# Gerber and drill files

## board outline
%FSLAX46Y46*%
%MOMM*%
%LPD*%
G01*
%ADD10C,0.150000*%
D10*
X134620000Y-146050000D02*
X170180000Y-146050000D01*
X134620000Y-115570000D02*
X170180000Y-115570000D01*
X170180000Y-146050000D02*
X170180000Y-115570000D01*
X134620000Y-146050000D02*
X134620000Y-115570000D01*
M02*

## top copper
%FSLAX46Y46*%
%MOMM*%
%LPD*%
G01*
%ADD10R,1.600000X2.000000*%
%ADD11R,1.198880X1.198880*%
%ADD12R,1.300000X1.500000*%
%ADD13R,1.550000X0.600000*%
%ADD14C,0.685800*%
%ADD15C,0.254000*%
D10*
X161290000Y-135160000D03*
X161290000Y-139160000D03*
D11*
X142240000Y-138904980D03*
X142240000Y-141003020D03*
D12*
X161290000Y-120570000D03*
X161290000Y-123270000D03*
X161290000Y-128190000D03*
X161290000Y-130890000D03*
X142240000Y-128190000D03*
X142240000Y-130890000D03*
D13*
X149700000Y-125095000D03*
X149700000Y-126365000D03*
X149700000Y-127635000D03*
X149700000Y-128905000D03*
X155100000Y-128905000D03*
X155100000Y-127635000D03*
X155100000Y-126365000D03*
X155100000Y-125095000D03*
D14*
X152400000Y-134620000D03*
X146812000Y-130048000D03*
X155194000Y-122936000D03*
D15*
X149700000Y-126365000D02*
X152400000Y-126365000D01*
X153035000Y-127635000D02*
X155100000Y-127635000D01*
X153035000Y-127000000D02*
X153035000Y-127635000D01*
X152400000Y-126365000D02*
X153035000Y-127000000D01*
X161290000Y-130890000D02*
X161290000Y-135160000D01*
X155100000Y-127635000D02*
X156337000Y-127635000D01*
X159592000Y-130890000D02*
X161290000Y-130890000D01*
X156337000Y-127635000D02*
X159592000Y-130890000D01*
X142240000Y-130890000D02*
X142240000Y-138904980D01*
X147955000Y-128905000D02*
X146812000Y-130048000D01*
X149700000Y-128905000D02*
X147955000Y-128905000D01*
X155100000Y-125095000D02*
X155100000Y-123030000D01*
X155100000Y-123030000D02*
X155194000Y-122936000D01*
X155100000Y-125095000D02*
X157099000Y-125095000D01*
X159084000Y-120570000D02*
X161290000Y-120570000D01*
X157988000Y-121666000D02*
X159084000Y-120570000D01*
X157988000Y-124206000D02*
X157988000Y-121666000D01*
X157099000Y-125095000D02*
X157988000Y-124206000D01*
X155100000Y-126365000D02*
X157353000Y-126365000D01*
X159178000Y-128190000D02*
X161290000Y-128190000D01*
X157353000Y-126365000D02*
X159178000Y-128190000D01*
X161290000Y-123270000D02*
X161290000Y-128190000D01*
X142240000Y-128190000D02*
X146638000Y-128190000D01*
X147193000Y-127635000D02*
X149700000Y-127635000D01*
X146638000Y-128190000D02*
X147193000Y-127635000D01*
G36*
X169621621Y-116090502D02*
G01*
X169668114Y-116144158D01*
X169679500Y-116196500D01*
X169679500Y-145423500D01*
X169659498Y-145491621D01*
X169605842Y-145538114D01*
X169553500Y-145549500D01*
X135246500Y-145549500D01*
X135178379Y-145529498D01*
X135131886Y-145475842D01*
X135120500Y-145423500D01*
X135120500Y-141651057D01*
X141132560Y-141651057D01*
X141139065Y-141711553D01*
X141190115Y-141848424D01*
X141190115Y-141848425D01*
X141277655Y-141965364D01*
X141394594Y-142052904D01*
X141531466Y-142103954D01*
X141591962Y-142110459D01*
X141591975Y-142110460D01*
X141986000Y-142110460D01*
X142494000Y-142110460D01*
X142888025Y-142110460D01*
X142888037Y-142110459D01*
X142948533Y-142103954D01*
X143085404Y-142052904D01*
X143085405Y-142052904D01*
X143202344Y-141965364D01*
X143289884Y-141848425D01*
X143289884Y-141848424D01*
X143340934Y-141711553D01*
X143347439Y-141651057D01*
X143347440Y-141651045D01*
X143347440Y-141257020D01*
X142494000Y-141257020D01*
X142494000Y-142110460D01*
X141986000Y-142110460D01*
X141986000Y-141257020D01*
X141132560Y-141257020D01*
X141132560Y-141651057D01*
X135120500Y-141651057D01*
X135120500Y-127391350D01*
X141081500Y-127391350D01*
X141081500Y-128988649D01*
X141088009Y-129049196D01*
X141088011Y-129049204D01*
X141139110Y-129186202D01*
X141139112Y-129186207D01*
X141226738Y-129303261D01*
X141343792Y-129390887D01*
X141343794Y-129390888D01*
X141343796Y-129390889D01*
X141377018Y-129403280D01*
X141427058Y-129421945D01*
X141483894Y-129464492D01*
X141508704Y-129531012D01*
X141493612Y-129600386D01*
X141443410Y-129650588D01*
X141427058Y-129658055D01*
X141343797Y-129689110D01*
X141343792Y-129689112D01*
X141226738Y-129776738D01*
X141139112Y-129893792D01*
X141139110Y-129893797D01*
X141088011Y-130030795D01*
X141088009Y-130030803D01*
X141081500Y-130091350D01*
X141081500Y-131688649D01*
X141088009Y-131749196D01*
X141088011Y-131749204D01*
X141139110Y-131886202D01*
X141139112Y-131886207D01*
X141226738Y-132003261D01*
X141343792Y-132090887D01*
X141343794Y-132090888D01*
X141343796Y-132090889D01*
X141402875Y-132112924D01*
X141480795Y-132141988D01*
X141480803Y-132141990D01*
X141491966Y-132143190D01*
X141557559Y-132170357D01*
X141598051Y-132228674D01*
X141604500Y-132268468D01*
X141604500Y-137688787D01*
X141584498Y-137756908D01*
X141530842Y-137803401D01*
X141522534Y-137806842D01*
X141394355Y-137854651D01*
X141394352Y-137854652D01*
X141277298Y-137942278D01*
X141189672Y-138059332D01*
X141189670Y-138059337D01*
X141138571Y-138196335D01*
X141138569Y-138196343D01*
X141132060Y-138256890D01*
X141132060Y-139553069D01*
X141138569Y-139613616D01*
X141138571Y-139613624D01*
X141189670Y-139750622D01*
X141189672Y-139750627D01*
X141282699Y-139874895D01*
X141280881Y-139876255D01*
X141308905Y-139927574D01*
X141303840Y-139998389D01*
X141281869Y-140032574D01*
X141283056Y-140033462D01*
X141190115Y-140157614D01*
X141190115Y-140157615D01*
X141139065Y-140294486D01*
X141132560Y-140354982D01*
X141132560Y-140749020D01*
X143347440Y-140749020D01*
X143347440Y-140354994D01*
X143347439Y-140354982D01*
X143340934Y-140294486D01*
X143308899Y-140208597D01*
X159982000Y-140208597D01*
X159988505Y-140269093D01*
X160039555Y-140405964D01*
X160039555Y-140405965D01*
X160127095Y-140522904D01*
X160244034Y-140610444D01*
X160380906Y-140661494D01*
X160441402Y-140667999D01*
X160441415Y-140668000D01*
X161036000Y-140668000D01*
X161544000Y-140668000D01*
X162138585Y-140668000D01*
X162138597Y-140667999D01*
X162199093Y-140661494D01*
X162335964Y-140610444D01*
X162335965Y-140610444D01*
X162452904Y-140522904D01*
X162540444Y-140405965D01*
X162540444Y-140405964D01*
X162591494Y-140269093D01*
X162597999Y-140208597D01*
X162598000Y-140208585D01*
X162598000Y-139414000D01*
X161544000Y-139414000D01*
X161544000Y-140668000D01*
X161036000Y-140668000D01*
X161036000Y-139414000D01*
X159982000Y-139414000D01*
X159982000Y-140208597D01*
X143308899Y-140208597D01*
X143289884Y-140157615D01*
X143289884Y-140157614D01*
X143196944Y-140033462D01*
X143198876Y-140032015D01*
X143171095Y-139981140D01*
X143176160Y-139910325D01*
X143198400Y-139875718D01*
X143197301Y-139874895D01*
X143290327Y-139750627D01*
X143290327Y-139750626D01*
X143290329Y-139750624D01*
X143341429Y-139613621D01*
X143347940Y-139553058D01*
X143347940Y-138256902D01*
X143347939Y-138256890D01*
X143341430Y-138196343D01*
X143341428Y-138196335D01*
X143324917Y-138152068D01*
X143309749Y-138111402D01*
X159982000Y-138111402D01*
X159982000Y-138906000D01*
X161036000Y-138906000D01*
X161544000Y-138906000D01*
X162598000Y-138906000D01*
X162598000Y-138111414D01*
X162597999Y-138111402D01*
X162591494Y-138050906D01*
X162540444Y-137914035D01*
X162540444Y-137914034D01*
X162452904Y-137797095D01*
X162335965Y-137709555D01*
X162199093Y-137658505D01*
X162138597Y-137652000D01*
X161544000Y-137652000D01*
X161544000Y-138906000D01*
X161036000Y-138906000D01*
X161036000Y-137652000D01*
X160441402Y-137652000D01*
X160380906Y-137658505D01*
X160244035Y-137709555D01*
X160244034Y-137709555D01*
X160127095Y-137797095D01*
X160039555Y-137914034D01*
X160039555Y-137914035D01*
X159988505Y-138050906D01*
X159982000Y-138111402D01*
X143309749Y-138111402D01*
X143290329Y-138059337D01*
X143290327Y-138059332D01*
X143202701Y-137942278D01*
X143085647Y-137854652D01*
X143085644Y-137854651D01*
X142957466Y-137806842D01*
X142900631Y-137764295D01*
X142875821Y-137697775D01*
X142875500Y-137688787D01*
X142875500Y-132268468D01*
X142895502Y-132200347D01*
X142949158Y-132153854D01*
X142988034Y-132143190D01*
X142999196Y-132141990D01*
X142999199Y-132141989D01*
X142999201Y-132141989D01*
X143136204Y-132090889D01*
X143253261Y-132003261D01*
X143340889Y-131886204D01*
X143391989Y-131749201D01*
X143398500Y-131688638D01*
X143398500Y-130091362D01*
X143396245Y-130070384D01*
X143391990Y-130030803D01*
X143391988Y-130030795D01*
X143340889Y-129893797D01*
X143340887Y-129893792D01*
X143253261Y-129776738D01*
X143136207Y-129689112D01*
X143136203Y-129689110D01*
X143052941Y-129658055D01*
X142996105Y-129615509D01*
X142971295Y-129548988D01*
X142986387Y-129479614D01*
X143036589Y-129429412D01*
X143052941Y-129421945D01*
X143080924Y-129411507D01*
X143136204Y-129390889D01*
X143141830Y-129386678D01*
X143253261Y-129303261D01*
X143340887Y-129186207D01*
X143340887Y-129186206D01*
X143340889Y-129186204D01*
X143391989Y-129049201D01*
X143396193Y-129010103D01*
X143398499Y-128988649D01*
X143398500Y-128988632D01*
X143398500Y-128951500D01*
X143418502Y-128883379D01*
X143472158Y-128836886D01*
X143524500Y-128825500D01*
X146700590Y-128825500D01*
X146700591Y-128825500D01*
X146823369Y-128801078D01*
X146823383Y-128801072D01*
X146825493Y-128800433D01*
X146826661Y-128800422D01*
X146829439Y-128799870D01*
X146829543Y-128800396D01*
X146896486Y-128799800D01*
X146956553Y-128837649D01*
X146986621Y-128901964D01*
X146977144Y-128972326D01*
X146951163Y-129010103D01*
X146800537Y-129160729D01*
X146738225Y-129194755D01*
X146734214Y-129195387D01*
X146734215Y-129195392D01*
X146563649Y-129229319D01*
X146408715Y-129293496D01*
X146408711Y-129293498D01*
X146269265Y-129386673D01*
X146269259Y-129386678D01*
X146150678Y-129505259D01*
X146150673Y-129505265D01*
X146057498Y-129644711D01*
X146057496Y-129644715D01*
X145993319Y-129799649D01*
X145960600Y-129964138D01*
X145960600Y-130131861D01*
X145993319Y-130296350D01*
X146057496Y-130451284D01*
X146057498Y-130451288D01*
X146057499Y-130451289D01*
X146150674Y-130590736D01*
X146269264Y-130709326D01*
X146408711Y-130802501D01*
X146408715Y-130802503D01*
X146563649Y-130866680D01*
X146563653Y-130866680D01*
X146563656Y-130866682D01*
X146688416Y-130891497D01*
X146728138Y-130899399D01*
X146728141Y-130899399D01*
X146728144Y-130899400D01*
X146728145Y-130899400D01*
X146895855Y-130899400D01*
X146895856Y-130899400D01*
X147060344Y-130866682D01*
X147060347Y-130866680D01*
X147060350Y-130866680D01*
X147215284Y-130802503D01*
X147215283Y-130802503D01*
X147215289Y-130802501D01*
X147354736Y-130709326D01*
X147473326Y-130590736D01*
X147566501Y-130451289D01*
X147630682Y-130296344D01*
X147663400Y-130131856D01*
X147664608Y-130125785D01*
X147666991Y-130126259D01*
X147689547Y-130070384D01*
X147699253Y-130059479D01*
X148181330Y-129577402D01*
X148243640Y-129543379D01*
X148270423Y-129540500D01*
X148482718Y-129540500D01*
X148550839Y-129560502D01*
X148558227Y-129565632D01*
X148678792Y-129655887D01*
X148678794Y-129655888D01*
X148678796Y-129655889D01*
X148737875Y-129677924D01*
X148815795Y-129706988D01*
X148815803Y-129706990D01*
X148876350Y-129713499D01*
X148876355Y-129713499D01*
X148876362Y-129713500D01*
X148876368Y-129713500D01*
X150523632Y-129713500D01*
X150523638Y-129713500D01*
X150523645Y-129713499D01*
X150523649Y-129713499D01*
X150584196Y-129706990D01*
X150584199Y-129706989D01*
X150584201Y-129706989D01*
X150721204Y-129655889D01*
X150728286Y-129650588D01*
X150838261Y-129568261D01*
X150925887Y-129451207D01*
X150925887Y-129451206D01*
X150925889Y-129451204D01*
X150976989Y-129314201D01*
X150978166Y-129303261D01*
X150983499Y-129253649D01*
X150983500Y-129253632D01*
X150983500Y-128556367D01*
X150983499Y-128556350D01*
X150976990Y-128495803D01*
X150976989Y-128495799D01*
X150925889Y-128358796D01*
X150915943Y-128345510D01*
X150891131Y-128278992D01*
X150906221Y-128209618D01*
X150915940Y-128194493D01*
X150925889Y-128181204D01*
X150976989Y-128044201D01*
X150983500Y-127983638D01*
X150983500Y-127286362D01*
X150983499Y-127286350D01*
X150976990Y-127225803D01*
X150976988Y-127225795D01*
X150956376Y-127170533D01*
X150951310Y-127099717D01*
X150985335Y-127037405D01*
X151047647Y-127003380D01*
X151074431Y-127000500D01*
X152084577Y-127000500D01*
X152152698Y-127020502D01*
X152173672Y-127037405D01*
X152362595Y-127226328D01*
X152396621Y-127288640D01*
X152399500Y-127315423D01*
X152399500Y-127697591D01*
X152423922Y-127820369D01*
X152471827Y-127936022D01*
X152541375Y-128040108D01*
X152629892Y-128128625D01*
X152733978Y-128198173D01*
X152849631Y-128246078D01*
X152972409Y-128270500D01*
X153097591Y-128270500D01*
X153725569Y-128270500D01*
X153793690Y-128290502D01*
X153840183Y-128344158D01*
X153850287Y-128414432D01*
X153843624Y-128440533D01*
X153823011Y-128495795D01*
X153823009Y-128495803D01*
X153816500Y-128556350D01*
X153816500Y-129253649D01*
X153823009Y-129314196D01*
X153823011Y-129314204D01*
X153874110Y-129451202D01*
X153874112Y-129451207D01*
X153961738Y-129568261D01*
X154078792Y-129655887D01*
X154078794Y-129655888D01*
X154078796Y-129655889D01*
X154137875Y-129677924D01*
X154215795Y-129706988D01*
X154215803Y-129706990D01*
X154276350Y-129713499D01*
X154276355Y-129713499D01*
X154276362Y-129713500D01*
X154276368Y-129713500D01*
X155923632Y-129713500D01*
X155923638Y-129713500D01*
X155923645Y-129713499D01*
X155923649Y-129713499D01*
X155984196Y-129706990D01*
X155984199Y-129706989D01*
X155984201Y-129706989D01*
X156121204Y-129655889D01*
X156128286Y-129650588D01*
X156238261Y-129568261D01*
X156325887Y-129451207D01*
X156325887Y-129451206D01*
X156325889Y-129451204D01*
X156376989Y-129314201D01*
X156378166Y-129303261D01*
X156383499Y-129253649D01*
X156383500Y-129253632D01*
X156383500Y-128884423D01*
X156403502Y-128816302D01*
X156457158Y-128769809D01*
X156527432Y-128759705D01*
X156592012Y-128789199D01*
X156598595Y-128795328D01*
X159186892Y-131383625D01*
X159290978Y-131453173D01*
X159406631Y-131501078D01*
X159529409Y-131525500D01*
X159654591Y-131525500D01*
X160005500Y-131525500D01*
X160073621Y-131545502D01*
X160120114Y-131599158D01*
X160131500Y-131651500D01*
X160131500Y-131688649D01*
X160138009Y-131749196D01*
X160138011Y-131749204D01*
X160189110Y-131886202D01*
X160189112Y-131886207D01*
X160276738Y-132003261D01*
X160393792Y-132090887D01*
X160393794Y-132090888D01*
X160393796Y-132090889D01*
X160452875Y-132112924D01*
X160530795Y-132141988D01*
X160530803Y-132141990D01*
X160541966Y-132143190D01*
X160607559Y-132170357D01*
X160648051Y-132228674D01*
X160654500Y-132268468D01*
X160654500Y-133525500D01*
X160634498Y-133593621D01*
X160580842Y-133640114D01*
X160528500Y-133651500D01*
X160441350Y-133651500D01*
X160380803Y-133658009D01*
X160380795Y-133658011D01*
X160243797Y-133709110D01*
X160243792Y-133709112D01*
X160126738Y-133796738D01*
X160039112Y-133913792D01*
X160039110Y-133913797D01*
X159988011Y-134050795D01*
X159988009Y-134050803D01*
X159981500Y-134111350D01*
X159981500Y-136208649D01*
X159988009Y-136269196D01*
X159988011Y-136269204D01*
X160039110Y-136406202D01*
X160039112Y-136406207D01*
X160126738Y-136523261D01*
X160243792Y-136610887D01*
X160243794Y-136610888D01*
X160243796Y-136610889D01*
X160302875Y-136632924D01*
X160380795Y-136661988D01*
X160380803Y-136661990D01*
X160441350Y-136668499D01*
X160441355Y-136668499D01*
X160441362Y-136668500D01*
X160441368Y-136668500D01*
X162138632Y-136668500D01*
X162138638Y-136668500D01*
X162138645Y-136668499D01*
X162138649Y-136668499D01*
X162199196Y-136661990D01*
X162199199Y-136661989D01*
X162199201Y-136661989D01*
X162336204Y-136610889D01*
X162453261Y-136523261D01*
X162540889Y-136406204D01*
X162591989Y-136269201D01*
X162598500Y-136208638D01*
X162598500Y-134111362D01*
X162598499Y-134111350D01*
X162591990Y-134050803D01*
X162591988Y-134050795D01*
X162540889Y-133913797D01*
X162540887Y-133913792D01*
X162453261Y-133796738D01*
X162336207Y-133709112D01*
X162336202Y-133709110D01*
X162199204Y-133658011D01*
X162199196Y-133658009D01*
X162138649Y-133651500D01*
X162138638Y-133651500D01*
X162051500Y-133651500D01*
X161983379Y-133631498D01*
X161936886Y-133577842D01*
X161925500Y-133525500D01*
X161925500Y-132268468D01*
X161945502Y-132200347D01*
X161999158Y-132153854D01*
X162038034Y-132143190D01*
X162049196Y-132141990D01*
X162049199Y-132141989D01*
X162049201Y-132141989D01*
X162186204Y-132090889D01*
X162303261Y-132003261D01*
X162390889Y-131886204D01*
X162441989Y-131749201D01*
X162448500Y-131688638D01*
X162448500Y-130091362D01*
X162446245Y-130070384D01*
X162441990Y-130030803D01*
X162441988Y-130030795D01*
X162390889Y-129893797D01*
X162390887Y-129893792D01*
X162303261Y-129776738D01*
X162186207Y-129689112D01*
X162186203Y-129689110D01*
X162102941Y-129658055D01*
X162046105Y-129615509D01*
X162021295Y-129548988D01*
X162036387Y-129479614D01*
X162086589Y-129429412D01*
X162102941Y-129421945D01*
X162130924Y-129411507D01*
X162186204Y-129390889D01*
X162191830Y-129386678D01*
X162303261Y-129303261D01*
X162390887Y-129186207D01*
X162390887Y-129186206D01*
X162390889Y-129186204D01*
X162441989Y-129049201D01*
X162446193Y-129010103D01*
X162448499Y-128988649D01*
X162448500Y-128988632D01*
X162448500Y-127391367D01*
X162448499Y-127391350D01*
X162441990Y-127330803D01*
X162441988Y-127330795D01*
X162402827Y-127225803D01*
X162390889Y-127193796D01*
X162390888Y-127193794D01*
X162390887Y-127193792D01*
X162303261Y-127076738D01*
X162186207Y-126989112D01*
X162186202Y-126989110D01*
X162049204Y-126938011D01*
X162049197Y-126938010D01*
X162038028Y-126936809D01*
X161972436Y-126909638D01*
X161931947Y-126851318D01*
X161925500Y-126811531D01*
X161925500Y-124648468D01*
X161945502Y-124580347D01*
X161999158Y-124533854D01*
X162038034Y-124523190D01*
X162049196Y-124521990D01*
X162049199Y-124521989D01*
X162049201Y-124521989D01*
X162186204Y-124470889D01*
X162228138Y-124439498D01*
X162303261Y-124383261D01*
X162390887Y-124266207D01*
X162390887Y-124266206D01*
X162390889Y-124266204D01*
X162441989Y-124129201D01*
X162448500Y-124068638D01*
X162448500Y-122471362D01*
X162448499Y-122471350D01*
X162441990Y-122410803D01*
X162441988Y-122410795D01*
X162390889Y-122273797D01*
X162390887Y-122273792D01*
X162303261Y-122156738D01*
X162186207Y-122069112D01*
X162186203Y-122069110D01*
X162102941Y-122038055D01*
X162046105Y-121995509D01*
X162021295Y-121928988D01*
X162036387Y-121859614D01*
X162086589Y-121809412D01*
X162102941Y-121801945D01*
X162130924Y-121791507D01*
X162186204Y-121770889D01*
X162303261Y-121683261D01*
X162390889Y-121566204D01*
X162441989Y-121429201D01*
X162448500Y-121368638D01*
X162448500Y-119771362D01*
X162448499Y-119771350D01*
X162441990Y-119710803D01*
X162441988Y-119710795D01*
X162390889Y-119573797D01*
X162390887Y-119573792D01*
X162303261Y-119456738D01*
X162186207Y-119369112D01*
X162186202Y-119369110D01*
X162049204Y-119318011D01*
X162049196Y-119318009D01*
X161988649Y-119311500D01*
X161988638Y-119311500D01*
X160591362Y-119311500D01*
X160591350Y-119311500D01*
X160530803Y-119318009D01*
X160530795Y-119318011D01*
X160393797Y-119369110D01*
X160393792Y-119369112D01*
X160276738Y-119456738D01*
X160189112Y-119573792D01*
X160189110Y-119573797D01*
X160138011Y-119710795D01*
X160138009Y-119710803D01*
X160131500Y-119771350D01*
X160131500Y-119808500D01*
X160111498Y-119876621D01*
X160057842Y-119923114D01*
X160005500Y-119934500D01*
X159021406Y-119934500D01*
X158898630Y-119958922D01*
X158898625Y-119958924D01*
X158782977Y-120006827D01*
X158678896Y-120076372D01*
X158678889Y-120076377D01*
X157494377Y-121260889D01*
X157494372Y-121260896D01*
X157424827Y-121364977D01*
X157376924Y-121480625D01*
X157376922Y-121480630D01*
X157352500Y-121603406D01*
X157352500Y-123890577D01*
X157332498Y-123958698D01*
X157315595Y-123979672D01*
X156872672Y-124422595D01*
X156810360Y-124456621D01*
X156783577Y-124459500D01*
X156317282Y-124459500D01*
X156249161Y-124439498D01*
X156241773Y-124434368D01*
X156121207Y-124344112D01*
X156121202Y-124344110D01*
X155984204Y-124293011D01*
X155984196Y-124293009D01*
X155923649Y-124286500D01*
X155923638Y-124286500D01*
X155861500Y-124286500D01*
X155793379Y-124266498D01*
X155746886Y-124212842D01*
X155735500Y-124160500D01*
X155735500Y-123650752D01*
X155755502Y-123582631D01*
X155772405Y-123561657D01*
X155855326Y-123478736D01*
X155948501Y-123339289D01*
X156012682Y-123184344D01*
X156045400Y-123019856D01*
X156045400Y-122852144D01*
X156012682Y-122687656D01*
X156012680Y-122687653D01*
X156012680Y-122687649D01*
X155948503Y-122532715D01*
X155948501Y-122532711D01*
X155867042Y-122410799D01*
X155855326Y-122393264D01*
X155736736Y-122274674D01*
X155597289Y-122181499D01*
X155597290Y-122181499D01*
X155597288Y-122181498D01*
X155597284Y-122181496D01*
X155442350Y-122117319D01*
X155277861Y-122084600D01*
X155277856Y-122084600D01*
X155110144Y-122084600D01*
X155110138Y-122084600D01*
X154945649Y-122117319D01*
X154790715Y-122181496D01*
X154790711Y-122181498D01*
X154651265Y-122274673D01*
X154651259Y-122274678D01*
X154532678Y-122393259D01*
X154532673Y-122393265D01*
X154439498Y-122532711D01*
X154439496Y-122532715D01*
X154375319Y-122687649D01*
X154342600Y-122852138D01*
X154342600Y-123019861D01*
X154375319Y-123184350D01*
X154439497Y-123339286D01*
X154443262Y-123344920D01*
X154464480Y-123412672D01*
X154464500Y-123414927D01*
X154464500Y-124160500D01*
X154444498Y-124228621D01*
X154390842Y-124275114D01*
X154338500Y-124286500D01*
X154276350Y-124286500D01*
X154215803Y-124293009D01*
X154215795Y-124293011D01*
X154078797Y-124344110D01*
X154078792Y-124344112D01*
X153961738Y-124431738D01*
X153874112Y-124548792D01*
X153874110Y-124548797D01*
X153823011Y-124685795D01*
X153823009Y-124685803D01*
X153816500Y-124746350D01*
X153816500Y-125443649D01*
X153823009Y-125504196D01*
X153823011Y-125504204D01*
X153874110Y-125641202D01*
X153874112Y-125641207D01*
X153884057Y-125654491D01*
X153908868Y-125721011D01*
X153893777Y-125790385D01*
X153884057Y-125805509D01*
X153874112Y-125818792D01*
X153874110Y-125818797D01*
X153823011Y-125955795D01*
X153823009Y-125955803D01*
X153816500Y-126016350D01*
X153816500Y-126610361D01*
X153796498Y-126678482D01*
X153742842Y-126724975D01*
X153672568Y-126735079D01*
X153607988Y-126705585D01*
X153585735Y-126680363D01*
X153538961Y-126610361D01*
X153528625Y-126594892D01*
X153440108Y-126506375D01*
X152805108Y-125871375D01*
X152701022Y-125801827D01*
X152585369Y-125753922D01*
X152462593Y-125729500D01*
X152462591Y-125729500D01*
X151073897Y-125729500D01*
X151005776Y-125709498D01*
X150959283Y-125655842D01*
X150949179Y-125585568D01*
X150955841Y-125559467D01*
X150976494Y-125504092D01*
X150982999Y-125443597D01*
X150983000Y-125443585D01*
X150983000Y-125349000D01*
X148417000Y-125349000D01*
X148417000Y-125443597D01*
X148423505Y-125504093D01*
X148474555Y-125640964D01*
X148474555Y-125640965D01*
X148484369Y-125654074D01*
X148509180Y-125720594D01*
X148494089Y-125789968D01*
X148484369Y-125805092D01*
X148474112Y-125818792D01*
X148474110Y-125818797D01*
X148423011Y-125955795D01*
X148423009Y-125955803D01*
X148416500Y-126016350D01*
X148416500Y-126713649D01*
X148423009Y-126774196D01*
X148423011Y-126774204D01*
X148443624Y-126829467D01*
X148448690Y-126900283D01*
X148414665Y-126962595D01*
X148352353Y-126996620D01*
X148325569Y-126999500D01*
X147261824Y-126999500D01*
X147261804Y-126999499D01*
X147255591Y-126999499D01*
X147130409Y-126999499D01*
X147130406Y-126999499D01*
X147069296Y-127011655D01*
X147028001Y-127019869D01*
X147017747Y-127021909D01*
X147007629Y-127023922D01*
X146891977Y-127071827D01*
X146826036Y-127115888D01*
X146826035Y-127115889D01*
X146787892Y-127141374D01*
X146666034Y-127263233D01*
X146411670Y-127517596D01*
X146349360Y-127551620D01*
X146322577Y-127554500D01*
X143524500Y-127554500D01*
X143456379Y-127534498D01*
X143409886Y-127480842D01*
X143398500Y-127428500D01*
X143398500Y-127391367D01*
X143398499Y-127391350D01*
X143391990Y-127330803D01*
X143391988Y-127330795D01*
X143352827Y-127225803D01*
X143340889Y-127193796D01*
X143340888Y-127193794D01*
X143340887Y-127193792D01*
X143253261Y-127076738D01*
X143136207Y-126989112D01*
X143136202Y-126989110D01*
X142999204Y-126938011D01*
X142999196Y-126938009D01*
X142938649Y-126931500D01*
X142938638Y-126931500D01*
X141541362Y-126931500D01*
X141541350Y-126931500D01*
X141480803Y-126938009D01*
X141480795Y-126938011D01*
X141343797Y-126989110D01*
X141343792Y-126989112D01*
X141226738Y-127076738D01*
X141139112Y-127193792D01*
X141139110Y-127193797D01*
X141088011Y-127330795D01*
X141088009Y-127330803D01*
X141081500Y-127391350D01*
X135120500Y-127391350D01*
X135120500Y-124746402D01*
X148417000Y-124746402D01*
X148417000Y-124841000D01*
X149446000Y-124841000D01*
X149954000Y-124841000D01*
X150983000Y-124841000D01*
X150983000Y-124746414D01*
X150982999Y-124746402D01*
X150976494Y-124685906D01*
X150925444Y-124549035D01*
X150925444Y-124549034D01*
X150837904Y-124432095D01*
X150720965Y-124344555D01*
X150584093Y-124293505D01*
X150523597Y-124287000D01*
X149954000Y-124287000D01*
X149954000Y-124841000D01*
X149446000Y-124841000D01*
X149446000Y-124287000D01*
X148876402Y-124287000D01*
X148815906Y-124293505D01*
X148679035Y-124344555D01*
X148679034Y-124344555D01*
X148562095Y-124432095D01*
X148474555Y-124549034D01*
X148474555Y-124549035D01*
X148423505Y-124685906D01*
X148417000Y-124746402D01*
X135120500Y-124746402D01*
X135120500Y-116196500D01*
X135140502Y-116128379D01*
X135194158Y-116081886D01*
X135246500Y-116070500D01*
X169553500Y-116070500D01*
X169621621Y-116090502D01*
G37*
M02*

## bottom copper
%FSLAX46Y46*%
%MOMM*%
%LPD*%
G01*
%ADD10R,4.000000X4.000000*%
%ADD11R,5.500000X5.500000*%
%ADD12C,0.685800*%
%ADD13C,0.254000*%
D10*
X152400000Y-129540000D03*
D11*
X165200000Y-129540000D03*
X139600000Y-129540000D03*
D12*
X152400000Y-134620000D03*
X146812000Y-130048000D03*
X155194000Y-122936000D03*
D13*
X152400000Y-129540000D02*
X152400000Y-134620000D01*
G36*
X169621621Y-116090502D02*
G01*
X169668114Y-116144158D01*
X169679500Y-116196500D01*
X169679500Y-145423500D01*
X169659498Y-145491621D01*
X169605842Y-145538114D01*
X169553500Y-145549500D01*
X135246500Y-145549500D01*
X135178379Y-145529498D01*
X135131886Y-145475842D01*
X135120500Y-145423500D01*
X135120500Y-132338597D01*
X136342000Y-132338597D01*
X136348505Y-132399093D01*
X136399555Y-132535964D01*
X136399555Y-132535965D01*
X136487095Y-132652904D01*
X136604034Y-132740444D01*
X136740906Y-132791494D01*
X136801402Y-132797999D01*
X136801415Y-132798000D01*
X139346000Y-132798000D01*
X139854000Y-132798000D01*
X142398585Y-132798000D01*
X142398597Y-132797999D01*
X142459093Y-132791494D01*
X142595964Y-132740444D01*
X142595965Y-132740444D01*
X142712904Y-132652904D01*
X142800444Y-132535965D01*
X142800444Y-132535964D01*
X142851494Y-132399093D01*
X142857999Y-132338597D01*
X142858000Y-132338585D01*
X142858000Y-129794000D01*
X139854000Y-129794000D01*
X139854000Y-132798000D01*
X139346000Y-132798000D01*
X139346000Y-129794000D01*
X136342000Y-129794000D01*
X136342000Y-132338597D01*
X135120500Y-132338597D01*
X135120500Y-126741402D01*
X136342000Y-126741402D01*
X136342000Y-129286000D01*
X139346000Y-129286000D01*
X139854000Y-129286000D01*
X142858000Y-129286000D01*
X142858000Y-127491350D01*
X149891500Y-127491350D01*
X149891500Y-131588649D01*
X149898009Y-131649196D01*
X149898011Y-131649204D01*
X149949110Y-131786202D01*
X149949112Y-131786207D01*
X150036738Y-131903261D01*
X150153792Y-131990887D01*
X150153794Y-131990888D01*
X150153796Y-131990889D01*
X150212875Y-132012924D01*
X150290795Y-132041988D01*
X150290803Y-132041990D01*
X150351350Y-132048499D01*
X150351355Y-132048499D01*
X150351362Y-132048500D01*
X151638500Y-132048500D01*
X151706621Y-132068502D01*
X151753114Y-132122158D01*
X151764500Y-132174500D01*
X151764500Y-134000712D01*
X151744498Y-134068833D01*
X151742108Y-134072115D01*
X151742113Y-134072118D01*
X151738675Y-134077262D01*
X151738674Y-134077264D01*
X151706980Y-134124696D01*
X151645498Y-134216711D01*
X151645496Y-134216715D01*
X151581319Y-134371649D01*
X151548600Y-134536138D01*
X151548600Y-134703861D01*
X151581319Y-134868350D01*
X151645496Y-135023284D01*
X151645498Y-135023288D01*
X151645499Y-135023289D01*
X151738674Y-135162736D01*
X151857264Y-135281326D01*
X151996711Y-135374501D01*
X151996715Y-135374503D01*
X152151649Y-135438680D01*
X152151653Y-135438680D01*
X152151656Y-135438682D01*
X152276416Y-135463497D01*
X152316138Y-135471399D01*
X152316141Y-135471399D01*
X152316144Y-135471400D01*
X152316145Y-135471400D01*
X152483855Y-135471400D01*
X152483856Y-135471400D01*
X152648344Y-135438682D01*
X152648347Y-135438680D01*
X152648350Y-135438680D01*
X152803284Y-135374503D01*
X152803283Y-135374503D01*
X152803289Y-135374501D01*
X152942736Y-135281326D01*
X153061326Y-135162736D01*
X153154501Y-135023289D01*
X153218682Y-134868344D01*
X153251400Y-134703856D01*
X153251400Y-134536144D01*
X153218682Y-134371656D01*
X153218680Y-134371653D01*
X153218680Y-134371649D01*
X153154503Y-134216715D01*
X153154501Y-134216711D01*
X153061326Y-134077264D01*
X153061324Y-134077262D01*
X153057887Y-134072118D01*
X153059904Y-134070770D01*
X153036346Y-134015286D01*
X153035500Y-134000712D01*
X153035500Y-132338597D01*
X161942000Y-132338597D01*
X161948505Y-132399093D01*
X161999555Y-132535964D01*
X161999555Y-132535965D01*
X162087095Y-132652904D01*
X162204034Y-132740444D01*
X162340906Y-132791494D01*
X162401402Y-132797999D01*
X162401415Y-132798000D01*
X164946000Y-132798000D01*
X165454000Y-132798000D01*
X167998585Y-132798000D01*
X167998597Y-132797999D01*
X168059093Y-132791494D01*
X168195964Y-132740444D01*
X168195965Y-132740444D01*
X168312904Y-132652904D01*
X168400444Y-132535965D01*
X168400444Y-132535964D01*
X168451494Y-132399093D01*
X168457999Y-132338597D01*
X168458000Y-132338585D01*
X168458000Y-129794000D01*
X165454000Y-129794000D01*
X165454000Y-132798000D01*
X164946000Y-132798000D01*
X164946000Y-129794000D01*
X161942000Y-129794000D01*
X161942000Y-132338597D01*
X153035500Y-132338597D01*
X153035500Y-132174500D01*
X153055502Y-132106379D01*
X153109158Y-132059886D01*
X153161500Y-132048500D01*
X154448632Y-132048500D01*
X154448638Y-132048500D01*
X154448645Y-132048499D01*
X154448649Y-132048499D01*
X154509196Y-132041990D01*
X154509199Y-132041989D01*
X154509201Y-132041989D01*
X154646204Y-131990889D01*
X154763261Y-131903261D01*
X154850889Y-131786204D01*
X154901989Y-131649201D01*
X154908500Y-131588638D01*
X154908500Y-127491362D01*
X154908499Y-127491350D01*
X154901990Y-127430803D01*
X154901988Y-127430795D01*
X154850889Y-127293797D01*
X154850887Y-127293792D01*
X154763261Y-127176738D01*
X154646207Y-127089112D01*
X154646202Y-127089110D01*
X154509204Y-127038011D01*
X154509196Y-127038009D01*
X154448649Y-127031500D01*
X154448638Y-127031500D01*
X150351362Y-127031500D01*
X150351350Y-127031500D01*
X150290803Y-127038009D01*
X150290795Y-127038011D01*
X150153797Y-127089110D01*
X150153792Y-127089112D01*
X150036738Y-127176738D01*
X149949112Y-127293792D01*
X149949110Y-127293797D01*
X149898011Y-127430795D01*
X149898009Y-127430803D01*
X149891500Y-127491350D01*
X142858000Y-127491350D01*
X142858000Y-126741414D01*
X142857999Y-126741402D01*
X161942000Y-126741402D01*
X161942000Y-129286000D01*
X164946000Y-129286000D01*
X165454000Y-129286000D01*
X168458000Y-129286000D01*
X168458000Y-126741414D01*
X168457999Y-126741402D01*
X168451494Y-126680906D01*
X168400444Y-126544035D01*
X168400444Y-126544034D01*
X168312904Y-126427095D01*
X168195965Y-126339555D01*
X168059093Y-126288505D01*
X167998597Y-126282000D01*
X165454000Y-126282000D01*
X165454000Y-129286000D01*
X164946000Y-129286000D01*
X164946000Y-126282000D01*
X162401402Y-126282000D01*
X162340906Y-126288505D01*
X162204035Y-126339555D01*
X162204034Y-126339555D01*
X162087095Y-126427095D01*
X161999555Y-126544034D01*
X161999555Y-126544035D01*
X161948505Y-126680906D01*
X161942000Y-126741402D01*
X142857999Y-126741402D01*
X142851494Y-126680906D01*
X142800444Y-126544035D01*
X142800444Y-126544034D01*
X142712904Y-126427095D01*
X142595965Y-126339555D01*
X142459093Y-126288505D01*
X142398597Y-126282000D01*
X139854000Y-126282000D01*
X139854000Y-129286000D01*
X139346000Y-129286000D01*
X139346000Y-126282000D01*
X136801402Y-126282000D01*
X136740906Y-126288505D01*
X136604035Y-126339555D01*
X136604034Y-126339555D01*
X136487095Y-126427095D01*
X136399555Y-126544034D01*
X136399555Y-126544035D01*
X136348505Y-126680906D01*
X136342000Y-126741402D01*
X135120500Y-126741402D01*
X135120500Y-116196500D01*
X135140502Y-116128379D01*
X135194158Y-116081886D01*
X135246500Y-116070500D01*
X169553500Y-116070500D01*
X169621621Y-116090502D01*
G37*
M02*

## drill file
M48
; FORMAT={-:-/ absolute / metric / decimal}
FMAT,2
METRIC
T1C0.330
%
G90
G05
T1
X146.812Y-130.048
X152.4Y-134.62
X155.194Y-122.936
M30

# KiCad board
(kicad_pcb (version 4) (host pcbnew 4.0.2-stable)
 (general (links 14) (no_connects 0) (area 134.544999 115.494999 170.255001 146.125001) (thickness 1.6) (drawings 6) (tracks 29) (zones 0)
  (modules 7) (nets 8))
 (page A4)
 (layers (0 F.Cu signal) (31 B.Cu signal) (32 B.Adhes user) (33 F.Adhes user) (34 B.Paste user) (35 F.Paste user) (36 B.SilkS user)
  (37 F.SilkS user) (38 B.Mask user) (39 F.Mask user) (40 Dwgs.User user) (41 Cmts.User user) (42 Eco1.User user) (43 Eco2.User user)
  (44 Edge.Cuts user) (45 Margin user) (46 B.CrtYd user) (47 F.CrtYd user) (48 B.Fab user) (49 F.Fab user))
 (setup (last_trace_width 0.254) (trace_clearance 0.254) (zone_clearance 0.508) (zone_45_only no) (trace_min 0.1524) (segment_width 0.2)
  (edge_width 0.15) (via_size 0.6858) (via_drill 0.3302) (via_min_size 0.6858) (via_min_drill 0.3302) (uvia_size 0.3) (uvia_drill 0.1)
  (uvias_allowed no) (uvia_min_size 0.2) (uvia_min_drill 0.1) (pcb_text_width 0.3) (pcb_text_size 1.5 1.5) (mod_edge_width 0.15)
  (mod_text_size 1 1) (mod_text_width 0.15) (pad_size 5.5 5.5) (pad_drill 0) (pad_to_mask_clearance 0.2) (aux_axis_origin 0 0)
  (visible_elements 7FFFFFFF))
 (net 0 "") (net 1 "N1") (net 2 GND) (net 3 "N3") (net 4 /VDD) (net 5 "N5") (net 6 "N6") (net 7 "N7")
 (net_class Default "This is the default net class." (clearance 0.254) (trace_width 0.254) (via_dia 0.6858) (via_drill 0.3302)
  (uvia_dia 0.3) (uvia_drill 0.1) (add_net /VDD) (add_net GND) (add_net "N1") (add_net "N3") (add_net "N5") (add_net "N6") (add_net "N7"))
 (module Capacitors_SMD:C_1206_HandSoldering (layer F.Cu) (at 161.29 137.16 270)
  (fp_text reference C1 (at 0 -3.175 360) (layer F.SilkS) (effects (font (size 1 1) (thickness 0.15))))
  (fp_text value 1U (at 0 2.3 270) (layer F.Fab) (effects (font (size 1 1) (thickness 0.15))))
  (pad 1 smd rect (at -2 0 270) (size 2 1.6) (layers F.Cu F.Paste F.Mask) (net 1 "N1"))
  (pad 2 smd rect (at 2 0 270) (size 2 1.6) (layers F.Cu F.Paste F.Mask) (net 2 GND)))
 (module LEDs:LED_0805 (layer F.Cu) (at 142.24 139.954 90)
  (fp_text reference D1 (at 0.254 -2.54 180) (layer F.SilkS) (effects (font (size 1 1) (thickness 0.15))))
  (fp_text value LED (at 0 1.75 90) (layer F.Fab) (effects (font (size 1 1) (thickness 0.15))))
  (pad 2 smd rect (at 1.04902 0 270) (size 1.19888 1.19888) (layers F.Cu F.Paste F.Mask) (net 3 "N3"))
  (pad 1 smd rect (at -1.04902 0 270) (size 1.19888 1.19888) (layers F.Cu F.Paste F.Mask) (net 2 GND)))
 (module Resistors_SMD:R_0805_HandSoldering (layer F.Cu) (at 161.29 121.92 270)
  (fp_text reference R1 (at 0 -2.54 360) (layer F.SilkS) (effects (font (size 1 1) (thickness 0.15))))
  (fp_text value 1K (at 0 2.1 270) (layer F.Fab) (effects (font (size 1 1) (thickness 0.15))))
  (pad 1 smd rect (at -1.35 0 270) (size 1.5 1.3) (layers F.Cu F.Paste F.Mask) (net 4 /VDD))
  (pad 2 smd rect (at 1.35 0 270) (size 1.5 1.3) (layers F.Cu F.Paste F.Mask) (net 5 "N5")))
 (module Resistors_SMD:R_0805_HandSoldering (layer F.Cu) (at 161.29 129.54 270)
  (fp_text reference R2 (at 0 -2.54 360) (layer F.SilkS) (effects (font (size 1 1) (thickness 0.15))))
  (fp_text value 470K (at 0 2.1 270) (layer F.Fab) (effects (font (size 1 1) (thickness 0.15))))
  (pad 1 smd rect (at -1.35 0 270) (size 1.5 1.3) (layers F.Cu F.Paste F.Mask) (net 5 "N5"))
  (pad 2 smd rect (at 1.35 0 270) (size 1.5 1.3) (layers F.Cu F.Paste F.Mask) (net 1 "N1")))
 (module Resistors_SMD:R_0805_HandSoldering (layer F.Cu) (at 142.24 129.54 270)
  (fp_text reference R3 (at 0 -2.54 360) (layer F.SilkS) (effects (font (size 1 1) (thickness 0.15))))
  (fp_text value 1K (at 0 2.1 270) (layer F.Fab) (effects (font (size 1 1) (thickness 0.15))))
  (pad 1 smd rect (at -1.35 0 270) (size 1.5 1.3) (layers F.Cu F.Paste F.Mask) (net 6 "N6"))
  (pad 2 smd rect (at 1.35 0 270) (size 1.5 1.3) (layers F.Cu F.Paste F.Mask) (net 3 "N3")))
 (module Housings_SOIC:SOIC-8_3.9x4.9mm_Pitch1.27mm (layer F.Cu) (at 152.4 127)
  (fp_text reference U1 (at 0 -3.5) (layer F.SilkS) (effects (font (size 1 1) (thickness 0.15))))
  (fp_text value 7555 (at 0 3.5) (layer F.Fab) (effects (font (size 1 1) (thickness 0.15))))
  (pad 1 smd rect (at -2.7 -1.905) (size 1.55 0.6) (layers F.Cu F.Paste F.Mask) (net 2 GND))
  (pad 2 smd rect (at -2.7 -0.635) (size 1.55 0.6) (layers F.Cu F.Paste F.Mask) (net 1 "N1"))
  (pad 3 smd rect (at -2.7 0.635) (size 1.55 0.6) (layers F.Cu F.Paste F.Mask) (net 6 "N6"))
  (pad 4 smd rect (at -2.7 1.905) (size 1.55 0.6) (layers F.Cu F.Paste F.Mask) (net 4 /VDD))
  (pad 5 smd rect (at 2.7 1.905) (size 1.55 0.6) (layers F.Cu F.Paste F.Mask) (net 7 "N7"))
  (pad 6 smd rect (at 2.7 0.635) (size 1.55 0.6) (layers F.Cu F.Paste F.Mask) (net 1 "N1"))
  (pad 7 smd rect (at 2.7 -0.635) (size 1.55 0.6) (layers F.Cu F.Paste F.Mask) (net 5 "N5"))
  (pad 8 smd rect (at 2.7 -1.905) (size 1.55 0.6) (layers F.Cu F.Paste F.Mask) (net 4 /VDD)))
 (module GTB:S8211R (layer B.Cu) (at 152.4 129.54 180)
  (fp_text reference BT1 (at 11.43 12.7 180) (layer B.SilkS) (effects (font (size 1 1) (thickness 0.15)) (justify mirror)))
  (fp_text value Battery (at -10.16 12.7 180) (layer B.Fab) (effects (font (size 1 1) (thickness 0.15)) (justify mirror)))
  (pad 2 smd rect (at 0 0 180) (size 4 4) (layers B.Cu B.Paste B.Mask) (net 2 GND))
  (pad 1 smd rect (at -12.8 0 180) (size 5.5 5.5) (layers B.Cu B.Paste B.Mask) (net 4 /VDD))
  (pad 1 smd rect (at 12.8 0 180) (size 5.5 5.5) (layers B.Cu B.Paste B.Mask) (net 4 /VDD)))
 (gr_line (start 134.62 146.05) (end 170.18 146.05) (angle 90) (layer Edge.Cuts) (width 0.15))
 (gr_line (start 134.62 115.57) (end 170.18 115.57) (angle 90) (layer Edge.Cuts) (width 0.15))
 (gr_line (start 170.18 146.05) (end 170.18 115.57) (angle 90) (layer Edge.Cuts) (width 0.15))
 (gr_line (start 134.62 146.05) (end 134.62 115.57) (angle 90) (layer Edge.Cuts) (width 0.15))
 (segment (start 149.7 126.365) (end 152.4 126.365) (width 0.254) (layer F.Cu) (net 1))
 (segment (start 153.035 127.635) (end 155.1 127.635) (width 0.254) (layer F.Cu) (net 1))
 (segment (start 153.035 127) (end 153.035 127.635) (width 0.254) (layer F.Cu) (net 1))
 (segment (start 152.4 126.365) (end 153.035 127) (width 0.254) (layer F.Cu) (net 1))
 (segment (start 161.29 130.89) (end 161.29 135.16) (width 0.254) (layer F.Cu) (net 1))
 (segment (start 155.1 127.635) (end 156.337 127.635) (width 0.254) (layer F.Cu) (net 1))
 (segment (start 159.592 130.89) (end 161.29 130.89) (width 0.254) (layer F.Cu) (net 1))
 (segment (start 156.337 127.635) (end 159.592 130.89) (width 0.254) (layer F.Cu) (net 1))
 (segment (start 152.4 129.54) (end 152.4 134.62) (width 0.254) (layer B.Cu) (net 2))
 (via (at 152.4 134.62) (size 0.6858) (drill 0.3302) (layers F.Cu B.Cu) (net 2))
 (segment (start 142.24 130.89) (end 142.24 138.90498) (width 0.254) (layer F.Cu) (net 3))
 (via (at 146.812 130.048) (size 0.6858) (drill 0.3302) (layers F.Cu B.Cu) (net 4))
 (segment (start 147.955 128.905) (end 146.812 130.048) (width 0.254) (layer F.Cu) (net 4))
 (segment (start 149.7 128.905) (end 147.955 128.905) (width 0.254) (layer F.Cu) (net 4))
 (segment (start 155.1 125.095) (end 155.1 123.03) (width 0.254) (layer F.Cu) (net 4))
 (via (at 155.194 122.936) (size 0.6858) (drill 0.3302) (layers F.Cu B.Cu) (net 4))
 (segment (start 155.1 123.03) (end 155.194 122.936) (width 0.254) (layer F.Cu) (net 4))
 (segment (start 155.1 125.095) (end 157.099 125.095) (width 0.254) (layer F.Cu) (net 4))
 (segment (start 159.084 120.57) (end 161.29 120.57) (width 0.254) (layer F.Cu) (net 4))
 (segment (start 157.988 121.666) (end 159.084 120.57) (width 0.254) (layer F.Cu) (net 4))
 (segment (start 157.988 124.206) (end 157.988 121.666) (width 0.254) (layer F.Cu) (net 4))
 (segment (start 157.099 125.095) (end 157.988 124.206) (width 0.254) (layer F.Cu) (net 4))
 (segment (start 155.1 126.365) (end 157.353 126.365) (width 0.254) (layer F.Cu) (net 5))
 (segment (start 159.178 128.19) (end 161.29 128.19) (width 0.254) (layer F.Cu) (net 5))
 (segment (start 157.353 126.365) (end 159.178 128.19) (width 0.254) (layer F.Cu) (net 5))
 (segment (start 161.29 123.27) (end 161.29 128.19) (width 0.254) (layer F.Cu) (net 5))
 (segment (start 142.24 128.19) (end 146.638 128.19) (width 0.254) (layer F.Cu) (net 6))
 (segment (start 147.193 127.635) (end 149.7 127.635) (width 0.254) (layer F.Cu) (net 6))
 (segment (start 146.638 128.19) (end 147.193 127.635) (width 0.254) (layer F.Cu) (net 6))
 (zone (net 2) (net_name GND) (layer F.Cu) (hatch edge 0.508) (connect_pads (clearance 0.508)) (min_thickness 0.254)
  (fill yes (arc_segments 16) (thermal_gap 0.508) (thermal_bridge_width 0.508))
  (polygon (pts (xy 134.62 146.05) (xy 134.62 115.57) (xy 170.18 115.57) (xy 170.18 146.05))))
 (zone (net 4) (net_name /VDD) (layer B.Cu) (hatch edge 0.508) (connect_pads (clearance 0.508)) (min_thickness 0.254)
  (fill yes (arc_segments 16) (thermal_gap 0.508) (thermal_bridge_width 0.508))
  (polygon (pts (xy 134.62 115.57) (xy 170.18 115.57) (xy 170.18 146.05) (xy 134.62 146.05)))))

